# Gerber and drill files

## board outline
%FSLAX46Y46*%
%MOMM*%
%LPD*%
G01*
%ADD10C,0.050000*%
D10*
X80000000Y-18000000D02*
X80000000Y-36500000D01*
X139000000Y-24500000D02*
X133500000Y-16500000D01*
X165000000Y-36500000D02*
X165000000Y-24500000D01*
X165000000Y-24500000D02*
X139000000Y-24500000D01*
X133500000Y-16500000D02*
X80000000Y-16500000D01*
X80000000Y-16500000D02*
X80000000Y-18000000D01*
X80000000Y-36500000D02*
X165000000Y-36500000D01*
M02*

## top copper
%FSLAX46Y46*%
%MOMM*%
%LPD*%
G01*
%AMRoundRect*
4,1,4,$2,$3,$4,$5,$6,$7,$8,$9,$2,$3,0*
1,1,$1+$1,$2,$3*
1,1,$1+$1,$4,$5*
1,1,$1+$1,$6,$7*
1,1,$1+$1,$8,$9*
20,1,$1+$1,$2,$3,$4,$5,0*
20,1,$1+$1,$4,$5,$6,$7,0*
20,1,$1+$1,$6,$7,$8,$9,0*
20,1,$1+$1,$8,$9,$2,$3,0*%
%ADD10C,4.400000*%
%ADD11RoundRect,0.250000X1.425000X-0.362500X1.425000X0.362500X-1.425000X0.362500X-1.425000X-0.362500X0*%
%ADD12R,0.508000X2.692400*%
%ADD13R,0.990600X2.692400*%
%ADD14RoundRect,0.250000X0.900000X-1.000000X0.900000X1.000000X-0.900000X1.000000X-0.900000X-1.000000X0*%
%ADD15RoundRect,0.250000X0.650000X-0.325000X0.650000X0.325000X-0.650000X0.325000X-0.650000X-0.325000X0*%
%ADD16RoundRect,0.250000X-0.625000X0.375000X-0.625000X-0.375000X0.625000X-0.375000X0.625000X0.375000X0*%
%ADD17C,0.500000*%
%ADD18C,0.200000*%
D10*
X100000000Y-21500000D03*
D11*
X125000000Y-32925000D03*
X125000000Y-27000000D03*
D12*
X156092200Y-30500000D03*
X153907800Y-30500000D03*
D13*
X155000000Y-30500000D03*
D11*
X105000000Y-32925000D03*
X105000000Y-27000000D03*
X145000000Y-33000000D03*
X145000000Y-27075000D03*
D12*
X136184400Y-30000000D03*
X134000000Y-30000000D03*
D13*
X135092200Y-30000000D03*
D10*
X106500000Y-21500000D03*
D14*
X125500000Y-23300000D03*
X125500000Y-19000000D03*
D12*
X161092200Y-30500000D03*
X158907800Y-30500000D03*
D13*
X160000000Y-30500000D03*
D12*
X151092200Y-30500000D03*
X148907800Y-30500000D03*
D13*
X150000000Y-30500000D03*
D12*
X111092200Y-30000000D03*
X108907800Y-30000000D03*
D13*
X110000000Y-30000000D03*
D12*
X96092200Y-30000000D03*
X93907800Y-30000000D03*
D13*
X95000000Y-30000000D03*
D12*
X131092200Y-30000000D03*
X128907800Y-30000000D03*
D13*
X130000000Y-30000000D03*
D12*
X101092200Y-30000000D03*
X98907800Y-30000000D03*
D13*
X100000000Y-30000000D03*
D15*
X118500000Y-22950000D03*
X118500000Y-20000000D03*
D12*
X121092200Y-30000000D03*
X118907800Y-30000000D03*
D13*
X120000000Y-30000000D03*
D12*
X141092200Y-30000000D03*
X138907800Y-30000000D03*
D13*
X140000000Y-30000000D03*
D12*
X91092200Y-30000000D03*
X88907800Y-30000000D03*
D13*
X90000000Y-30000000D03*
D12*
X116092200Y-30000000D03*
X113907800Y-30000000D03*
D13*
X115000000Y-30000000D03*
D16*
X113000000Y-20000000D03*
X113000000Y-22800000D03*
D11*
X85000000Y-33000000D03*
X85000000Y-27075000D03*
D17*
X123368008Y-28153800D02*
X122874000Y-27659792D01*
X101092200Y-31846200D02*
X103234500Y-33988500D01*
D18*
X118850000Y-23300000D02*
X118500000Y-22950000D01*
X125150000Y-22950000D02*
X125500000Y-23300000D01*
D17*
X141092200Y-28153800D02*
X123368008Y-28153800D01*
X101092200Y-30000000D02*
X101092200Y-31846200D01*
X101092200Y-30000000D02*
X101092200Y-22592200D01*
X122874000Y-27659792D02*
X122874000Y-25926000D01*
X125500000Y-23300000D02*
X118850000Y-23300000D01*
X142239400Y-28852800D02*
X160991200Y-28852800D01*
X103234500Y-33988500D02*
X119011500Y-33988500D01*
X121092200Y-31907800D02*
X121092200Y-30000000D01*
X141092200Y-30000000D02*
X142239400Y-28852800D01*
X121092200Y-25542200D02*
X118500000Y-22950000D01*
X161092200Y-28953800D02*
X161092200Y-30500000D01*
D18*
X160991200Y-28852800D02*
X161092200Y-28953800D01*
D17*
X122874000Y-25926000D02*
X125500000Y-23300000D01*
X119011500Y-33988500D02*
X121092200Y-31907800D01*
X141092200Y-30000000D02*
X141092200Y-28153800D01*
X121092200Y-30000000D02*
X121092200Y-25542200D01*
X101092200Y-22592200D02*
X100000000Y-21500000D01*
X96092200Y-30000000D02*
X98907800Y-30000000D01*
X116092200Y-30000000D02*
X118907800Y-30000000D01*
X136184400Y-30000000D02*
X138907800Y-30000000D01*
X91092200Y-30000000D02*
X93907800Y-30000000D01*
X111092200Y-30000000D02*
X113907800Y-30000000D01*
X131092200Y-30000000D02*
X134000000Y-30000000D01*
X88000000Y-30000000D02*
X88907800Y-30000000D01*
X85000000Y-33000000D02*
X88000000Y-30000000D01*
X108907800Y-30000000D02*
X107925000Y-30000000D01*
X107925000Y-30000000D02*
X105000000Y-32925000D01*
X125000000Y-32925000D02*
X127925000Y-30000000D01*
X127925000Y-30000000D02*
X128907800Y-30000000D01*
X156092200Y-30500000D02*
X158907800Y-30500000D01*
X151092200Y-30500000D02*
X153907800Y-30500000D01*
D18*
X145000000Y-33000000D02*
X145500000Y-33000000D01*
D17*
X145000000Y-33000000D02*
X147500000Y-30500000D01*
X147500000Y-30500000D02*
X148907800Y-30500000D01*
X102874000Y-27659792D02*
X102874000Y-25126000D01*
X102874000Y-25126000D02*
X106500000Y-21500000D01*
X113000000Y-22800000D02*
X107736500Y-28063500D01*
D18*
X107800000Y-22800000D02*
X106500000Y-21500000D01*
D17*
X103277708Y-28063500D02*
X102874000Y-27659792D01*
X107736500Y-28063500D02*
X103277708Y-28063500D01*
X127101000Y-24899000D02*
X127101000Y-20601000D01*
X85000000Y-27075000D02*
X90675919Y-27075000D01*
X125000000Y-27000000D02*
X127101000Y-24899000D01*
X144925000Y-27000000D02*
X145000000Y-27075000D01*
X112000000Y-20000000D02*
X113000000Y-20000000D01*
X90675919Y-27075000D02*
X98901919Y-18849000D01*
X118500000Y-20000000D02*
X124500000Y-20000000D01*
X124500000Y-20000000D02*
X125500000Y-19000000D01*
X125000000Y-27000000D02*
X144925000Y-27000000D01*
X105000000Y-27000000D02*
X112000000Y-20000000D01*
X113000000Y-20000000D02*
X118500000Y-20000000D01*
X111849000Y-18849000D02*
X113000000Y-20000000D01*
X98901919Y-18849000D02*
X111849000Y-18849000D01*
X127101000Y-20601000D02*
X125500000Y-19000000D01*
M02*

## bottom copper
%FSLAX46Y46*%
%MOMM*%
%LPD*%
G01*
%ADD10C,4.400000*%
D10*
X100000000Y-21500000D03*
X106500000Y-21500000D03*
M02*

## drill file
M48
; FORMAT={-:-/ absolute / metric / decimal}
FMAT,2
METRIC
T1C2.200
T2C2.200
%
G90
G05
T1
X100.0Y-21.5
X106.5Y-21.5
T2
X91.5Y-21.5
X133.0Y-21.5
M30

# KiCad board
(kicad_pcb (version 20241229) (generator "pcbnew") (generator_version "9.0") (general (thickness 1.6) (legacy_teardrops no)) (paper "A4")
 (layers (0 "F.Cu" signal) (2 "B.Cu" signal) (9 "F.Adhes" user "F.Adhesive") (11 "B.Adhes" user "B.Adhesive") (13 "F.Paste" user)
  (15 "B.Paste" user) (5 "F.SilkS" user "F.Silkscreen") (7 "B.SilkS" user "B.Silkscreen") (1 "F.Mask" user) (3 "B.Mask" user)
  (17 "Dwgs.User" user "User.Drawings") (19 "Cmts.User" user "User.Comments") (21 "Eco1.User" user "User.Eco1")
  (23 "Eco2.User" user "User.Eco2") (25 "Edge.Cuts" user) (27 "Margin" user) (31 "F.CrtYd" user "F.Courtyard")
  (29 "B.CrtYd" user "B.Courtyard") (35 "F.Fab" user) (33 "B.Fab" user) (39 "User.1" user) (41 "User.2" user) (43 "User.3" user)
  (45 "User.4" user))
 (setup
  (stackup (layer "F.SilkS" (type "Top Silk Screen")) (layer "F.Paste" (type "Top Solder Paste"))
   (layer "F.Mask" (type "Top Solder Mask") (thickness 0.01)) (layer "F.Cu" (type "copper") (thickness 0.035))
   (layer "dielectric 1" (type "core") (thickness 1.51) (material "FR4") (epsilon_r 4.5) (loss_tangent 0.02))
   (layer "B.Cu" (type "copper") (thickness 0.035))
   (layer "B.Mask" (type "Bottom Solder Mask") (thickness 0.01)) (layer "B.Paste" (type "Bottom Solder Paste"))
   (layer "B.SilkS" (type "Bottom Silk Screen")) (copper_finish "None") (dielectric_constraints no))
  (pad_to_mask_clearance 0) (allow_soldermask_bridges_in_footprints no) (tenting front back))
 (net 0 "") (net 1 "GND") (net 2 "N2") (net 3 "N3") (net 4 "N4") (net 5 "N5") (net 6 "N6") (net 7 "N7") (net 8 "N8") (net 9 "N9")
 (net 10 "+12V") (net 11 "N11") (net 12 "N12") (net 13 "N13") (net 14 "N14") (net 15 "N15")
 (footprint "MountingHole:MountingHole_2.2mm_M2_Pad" (layer "F.Cu") (at 100 21.5)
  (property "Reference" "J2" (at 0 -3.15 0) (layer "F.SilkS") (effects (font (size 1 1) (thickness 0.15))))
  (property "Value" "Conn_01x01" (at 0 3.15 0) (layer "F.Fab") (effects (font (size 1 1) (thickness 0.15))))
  (pad "1" thru_hole circle (at 0 0) (size 4.4 4.4) (drill 2.2) (layers "*.Cu" "*.Mask") (remove_unused_layers no) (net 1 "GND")
   (zone_connect 2)))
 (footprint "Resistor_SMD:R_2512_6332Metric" (layer "F.Cu") (at 125 29.9625 90)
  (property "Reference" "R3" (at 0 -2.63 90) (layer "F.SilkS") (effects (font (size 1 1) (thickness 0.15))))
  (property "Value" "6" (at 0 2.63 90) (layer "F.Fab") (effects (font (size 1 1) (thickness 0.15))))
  (pad "1" smd roundrect (at -2.9625 0 90) (size 1.225 3.35) (layers "F.Cu" "F.Mask" "F.Paste") (roundrect_rratio 0.204082) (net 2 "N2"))
  (pad "2" smd roundrect (at 2.9625 0 90) (size 1.225 3.35) (layers "F.Cu" "F.Mask" "F.Paste") (roundrect_rratio 0.204082) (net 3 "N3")))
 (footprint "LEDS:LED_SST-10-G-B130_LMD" (layer "F.Cu") (at 155 30.5 180)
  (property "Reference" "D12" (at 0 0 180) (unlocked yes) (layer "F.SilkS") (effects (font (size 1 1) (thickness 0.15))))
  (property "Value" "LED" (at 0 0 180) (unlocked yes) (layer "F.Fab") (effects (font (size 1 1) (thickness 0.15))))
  (pad "1" smd rect (at -1.0922 0 180) (size 0.508 2.6924) (layers "F.Cu" "F.Mask" "F.Paste") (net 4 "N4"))
  (pad "2" smd rect (at 1.0922 0 180) (size 0.508 2.6924) (layers "F.Cu" "F.Mask" "F.Paste") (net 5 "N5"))
  (pad "3" smd rect (at 0 0 180) (size 0.9906 2.6924) (layers "F.Cu" "F.Mask" "F.Paste")))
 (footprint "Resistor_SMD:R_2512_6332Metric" (layer "F.Cu") (at 105 29.9625 90)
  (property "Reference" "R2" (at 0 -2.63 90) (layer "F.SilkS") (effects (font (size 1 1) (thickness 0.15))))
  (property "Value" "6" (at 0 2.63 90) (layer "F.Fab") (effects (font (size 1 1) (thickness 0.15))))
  (pad "1" smd roundrect (at -2.9625 0 90) (size 1.225 3.35) (layers "F.Cu" "F.Mask" "F.Paste") (roundrect_rratio 0.204082) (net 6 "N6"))
  (pad "2" smd roundrect (at 2.9625 0 90) (size 1.225 3.35) (layers "F.Cu" "F.Mask" "F.Paste") (roundrect_rratio 0.204082) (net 3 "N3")))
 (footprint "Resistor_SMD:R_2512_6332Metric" (layer "F.Cu") (at 145 30.0375 90)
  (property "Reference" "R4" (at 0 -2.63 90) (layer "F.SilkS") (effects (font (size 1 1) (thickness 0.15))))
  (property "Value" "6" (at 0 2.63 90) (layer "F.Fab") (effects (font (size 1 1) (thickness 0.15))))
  (pad "1" smd roundrect (at -2.9625 0 90) (size 1.225 3.35) (layers "F.Cu" "F.Mask" "F.Paste") (roundrect_rratio 0.204082) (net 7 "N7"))
  (pad "2" smd roundrect (at 2.9625 0 90) (size 1.225 3.35) (layers "F.Cu" "F.Mask" "F.Paste") (roundrect_rratio 0.204082) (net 3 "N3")))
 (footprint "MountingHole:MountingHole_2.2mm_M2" (layer "F.Cu") (at 133 21.5)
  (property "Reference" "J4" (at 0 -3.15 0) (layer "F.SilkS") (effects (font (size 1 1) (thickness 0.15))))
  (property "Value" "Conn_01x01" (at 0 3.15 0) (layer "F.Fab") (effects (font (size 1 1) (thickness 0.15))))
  (pad "" np_thru_hole circle (at 0 0) (size 2.2 2.2) (drill 2.2) (layers "*.Cu" "*.Mask")))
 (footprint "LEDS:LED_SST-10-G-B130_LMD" (layer "F.Cu") (at 135.0922 30 180)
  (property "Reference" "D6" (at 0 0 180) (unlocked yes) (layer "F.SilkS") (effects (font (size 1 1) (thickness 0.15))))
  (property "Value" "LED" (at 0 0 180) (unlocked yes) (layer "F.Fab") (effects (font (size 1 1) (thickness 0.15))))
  (pad "1" smd rect (at -1.0922 0 180) (size 0.508 2.6924) (layers "F.Cu" "F.Mask" "F.Paste") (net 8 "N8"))
  (pad "2" smd rect (at 1.0922 0 180) (size 0.508 2.6924) (layers "F.Cu" "F.Mask" "F.Paste") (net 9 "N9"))
  (pad "3" smd rect (at 0 0 180) (size 0.9906 2.6924) (layers "F.Cu" "F.Mask" "F.Paste")))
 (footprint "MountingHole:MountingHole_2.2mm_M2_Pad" (layer "F.Cu") (at 106.5 21.5)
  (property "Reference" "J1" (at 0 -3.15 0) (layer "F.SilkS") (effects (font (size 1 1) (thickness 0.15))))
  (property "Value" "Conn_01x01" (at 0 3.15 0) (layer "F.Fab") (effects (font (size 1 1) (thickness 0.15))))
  (pad "1" thru_hole circle (at 0 0) (size 4.4 4.4) (drill 2.2) (layers "*.Cu" "*.Mask") (remove_unused_layers no) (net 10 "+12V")
   (zone_connect 2)))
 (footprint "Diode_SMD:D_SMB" (layer "F.Cu") (at 125.5 21.15 90)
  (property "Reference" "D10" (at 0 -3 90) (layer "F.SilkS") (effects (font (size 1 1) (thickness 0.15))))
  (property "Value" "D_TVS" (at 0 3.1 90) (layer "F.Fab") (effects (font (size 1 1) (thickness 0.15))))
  (pad "1" smd roundrect (at -2.15 0 90) (size 2.5 2.3) (layers "F.Cu" "F.Mask" "F.Paste") (roundrect_rratio 0.1086956522) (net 1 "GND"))
  (pad "2" smd roundrect (at 2.15 0 90) (size 2.5 2.3) (layers "F.Cu" "F.Mask" "F.Paste") (roundrect_rratio 0.1086956522) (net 3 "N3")))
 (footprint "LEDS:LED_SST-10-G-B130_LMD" (layer "F.Cu") (at 160 30.5 180)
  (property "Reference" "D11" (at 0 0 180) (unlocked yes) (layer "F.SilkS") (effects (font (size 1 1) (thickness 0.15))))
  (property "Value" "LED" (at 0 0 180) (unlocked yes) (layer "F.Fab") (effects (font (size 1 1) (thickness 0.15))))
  (pad "1" smd rect (at -1.0922 0 180) (size 0.508 2.6924) (layers "F.Cu" "F.Mask" "F.Paste") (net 1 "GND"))
  (pad "2" smd rect (at 1.0922 0 180) (size 0.508 2.6924) (layers "F.Cu" "F.Mask" "F.Paste") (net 4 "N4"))
  (pad "3" smd rect (at 0 0 180) (size 0.9906 2.6924) (layers "F.Cu" "F.Mask" "F.Paste")))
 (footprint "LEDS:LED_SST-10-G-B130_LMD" (layer "F.Cu") (at 150 30.5 180)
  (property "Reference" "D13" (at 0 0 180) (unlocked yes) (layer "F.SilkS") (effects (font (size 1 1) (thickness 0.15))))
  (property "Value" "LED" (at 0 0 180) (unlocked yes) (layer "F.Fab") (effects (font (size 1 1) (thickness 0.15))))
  (pad "1" smd rect (at -1.0922 0 180) (size 0.508 2.6924) (layers "F.Cu" "F.Mask" "F.Paste") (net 5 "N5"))
  (pad "2" smd rect (at 1.0922 0 180) (size 0.508 2.6924) (layers "F.Cu" "F.Mask" "F.Paste") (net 7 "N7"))
  (pad "3" smd rect (at 0 0 180) (size 0.9906 2.6924) (layers "F.Cu" "F.Mask" "F.Paste")))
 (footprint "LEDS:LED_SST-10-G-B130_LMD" (layer "F.Cu") (at 110 30 180)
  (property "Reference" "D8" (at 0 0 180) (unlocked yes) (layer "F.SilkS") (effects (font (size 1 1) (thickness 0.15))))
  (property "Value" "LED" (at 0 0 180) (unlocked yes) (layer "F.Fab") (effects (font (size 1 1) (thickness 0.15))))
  (pad "1" smd rect (at -1.0922 0 180) (size 0.508 2.6924) (layers "F.Cu" "F.Mask" "F.Paste") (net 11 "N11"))
  (pad "2" smd rect (at 1.0922 0 180) (size 0.508 2.6924) (layers "F.Cu" "F.Mask" "F.Paste") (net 6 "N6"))
  (pad "3" smd rect (at 0 0 180) (size 0.9906 2.6924) (layers "F.Cu" "F.Mask" "F.Paste")))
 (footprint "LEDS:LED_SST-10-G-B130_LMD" (layer "F.Cu") (at 95 30 180)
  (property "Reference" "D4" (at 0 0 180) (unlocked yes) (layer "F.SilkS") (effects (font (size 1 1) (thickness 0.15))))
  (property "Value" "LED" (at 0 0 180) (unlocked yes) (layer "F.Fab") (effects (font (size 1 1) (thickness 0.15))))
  (pad "1" smd rect (at -1.0922 0 180) (size 0.508 2.6924) (layers "F.Cu" "F.Mask" "F.Paste") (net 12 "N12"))
  (pad "2" smd rect (at 1.0922 0 180) (size 0.508 2.6924) (layers "F.Cu" "F.Mask" "F.Paste") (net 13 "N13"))
  (pad "3" smd rect (at 0 0 180) (size 0.9906 2.6924) (layers "F.Cu" "F.Mask" "F.Paste")))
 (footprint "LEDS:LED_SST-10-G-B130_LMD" (layer "F.Cu") (at 130 30 180)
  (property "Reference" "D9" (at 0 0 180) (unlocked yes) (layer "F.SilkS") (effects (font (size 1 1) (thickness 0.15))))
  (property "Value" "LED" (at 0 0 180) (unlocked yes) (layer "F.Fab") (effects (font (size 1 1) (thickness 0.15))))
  (pad "1" smd rect (at -1.0922 0 180) (size 0.508 2.6924) (layers "F.Cu" "F.Mask" "F.Paste") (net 9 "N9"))
  (pad "2" smd rect (at 1.0922 0 180) (size 0.508 2.6924) (layers "F.Cu" "F.Mask" "F.Paste") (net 2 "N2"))
  (pad "3" smd rect (at 0 0 180) (size 0.9906 2.6924) (layers "F.Cu" "F.Mask" "F.Paste")))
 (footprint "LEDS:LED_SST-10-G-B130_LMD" (layer "F.Cu") (at 100 30 180)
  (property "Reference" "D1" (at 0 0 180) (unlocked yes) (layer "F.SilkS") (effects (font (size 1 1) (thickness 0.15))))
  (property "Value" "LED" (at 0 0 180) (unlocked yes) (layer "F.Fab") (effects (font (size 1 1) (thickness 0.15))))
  (pad "1" smd rect (at -1.0922 0 180) (size 0.508 2.6924) (layers "F.Cu" "F.Mask" "F.Paste") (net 1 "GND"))
  (pad "2" smd rect (at 1.0922 0 180) (size 0.508 2.6924) (layers "F.Cu" "F.Mask" "F.Paste") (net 12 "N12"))
  (pad "3" smd rect (at 0 0 180) (size 0.9906 2.6924) (layers "F.Cu" "F.Mask" "F.Paste")))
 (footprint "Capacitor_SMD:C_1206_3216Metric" (layer "F.Cu") (at 118.5 21.475 90)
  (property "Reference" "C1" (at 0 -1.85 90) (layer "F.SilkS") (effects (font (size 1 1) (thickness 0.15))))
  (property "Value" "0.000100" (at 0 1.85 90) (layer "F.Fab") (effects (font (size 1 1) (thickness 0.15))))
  (pad "1" smd roundrect (at -1.475 0 90) (size 1.15 1.8) (layers "F.Cu" "F.Mask" "F.Paste") (roundrect_rratio 0.217391) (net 1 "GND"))
  (pad "2" smd roundrect (at 1.475 0 90) (size 1.15 1.8) (layers "F.Cu" "F.Mask" "F.Paste") (roundrect_rratio 0.217391) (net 3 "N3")))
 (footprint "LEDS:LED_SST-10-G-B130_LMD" (layer "F.Cu") (at 120 30 180)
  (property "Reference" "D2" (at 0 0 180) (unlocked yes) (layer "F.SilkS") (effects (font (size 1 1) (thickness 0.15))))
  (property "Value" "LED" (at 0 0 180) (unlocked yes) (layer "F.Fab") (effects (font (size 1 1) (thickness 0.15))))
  (pad "1" smd rect (at -1.0922 0 180) (size 0.508 2.6924) (layers "F.Cu" "F.Mask" "F.Paste") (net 1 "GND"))
  (pad "2" smd rect (at 1.0922 0 180) (size 0.508 2.6924) (layers "F.Cu" "F.Mask" "F.Paste") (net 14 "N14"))
  (pad "3" smd rect (at 0 0 180) (size 0.9906 2.6924) (layers "F.Cu" "F.Mask" "F.Paste")))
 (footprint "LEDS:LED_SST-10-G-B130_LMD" (layer "F.Cu") (at 140 30 180)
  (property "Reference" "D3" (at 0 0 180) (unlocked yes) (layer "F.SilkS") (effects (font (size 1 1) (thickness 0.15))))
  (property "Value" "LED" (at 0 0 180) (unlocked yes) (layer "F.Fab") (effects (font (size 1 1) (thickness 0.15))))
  (pad "1" smd rect (at -1.0922 0 180) (size 0.508 2.6924) (layers "F.Cu" "F.Mask" "F.Paste") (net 1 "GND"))
  (pad "2" smd rect (at 1.0922 0 180) (size 0.508 2.6924) (layers "F.Cu" "F.Mask" "F.Paste") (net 8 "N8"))
  (pad "3" smd rect (at 0 0 180) (size 0.9906 2.6924) (layers "F.Cu" "F.Mask" "F.Paste")))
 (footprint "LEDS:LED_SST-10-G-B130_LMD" (layer "F.Cu") (at 90 30 180)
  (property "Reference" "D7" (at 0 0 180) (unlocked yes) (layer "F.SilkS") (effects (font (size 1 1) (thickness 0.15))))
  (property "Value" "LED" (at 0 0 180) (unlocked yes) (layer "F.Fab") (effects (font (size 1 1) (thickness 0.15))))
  (pad "1" smd rect (at -1.0922 0 180) (size 0.508 2.6924) (layers "F.Cu" "F.Mask" "F.Paste") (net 13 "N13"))
  (pad "2" smd rect (at 1.0922 0 180) (size 0.508 2.6924) (layers "F.Cu" "F.Mask" "F.Paste") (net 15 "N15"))
  (pad "3" smd rect (at 0 0 180) (size 0.9906 2.6924) (layers "F.Cu" "F.Mask" "F.Paste")))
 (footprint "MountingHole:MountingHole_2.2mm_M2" (layer "F.Cu") (at 91.5 21.5)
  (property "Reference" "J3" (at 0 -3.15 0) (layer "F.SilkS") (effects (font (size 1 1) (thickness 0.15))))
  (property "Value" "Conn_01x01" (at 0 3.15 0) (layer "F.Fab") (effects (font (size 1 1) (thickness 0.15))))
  (pad "" np_thru_hole circle (at 0 0) (size 2.2 2.2) (drill 2.2) (layers "*.Cu" "*.Mask")))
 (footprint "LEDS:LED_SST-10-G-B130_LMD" (layer "F.Cu") (at 115 30 180)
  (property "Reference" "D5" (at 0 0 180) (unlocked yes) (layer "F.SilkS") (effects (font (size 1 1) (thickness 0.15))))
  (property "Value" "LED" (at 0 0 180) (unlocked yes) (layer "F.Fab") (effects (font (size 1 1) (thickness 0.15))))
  (pad "1" smd rect (at -1.0922 0 180) (size 0.508 2.6924) (layers "F.Cu" "F.Mask" "F.Paste") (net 14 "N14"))
  (pad "2" smd rect (at 1.0922 0 180) (size 0.508 2.6924) (layers "F.Cu" "F.Mask" "F.Paste") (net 11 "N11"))
  (pad "3" smd rect (at 0 0 180) (size 0.9906 2.6924) (layers "F.Cu" "F.Mask" "F.Paste")))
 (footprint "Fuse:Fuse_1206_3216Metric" (layer "F.Cu") (at 113 21.4 -90)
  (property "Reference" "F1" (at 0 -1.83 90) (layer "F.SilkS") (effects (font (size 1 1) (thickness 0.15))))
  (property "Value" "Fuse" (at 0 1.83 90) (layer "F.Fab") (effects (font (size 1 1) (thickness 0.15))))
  (pad "1" smd roundrect (at -1.4 0 270) (size 1.25 1.75) (layers "F.Cu" "F.Mask" "F.Paste") (roundrect_rratio 0.2) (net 3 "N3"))
  (pad "2" smd roundrect (at 1.4 0 270) (size 1.25 1.75) (layers "F.Cu" "F.Mask" "F.Paste") (roundrect_rratio 0.2) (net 10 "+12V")))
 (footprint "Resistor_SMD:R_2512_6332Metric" (layer "F.Cu") (at 85 30.0375 90)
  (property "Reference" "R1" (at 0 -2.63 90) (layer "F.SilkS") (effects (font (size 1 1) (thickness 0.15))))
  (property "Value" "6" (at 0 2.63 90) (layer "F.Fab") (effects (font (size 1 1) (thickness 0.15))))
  (pad "1" smd roundrect (at -2.9625 0 90) (size 1.225 3.35) (layers "F.Cu" "F.Mask" "F.Paste") (roundrect_rratio 0.204082) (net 15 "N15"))
  (pad "2" smd roundrect (at 2.9625 0 90) (size 1.225 3.35) (layers "F.Cu" "F.Mask" "F.Paste") (roundrect_rratio 0.204082) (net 3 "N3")))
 (gr_line (start 80 18) (end 80 36.5) (stroke (width 0.05) (type default)) (layer "Edge.Cuts"))
 (gr_line (start 139 24.5) (end 133.5 16.5) (stroke (width 0.05) (type default)) (layer "Edge.Cuts"))
 (gr_line (start 165 36.5) (end 165 24.5) (stroke (width 0.05) (type default)) (layer "Edge.Cuts"))
 (gr_line (start 165 24.5) (end 139 24.5) (stroke (width 0.05) (type default)) (layer "Edge.Cuts"))
 (gr_line (start 133.5 16.5) (end 80 16.5) (stroke (width 0.05) (type default)) (layer "Edge.Cuts"))
 (gr_line (start 80 16.5) (end 80 18) (stroke (width 0.05) (type default)) (layer "Edge.Cuts"))
 (gr_line (start 80 36.5) (end 165 36.5) (stroke (width 0.05) (type default)) (layer "Edge.Cuts"))
 (segment (start 123.368008 28.1538) (end 122.874 27.659792) (width 0.5) (layer "F.Cu") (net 1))
 (segment (start 101.0922 31.8462) (end 103.2345 33.9885) (width 0.5) (layer "F.Cu") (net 1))
 (segment (start 118.85 23.3) (end 118.5 22.95) (width 0.2) (layer "F.Cu") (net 1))
 (segment (start 125.15 22.95) (end 125.5 23.3) (width 0.2) (layer "F.Cu") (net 1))
 (segment (start 141.0922 28.1538) (end 123.368008 28.1538) (width 0.5) (layer "F.Cu") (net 1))
 (segment (start 101.0922 30) (end 101.0922 31.8462) (width 0.5) (layer "F.Cu") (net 1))
 (segment (start 101.0922 30) (end 101.0922 22.5922) (width 0.5) (layer "F.Cu") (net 1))
 (segment (start 122.874 27.659792) (end 122.874 25.926) (width 0.5) (layer "F.Cu") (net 1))
 (segment (start 125.5 23.3) (end 118.85 23.3) (width 0.5) (layer "F.Cu") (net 1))
 (segment (start 142.2394 28.8528) (end 160.9912 28.8528) (width 0.5) (layer "F.Cu") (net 1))
 (segment (start 103.2345 33.9885) (end 119.0115 33.9885) (width 0.5) (layer "F.Cu") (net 1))
 (segment (start 121.0922 31.9078) (end 121.0922 30) (width 0.5) (layer "F.Cu") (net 1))
 (segment (start 141.0922 30) (end 142.2394 28.8528) (width 0.5) (layer "F.Cu") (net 1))
 (segment (start 121.0922 25.5422) (end 118.5 22.95) (width 0.5) (layer "F.Cu") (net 1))
 (segment (start 161.0922 28.9538) (end 161.0922 30.5) (width 0.5) (layer "F.Cu") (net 1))
 (segment (start 160.9912 28.8528) (end 161.0922 28.9538) (width 0.2) (layer "F.Cu") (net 1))
 (segment (start 122.874 25.926) (end 125.5 23.3) (width 0.5) (layer "F.Cu") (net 1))
 (segment (start 119.0115 33.9885) (end 121.0922 31.9078) (width 0.5) (layer "F.Cu") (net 1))
 (segment (start 141.0922 30) (end 141.0922 28.1538) (width 0.5) (layer "F.Cu") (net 1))
 (segment (start 121.0922 30) (end 121.0922 25.5422) (width 0.5) (layer "F.Cu") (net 1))
 (segment (start 101.0922 22.5922) (end 100 21.5) (width 0.5) (layer "F.Cu") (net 1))
 (segment (start 96.0922 30) (end 98.9078 30) (width 0.5) (layer "F.Cu") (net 12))
 (segment (start 116.0922 30) (end 118.9078 30) (width 0.5) (layer "F.Cu") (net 14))
 (segment (start 136.1844 30) (end 138.9078 30) (width 0.5) (layer "F.Cu") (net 8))
 (segment (start 91.0922 30) (end 93.9078 30) (width 0.5) (layer "F.Cu") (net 13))
 (segment (start 111.0922 30) (end 113.9078 30) (width 0.5) (layer "F.Cu") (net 11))
 (segment (start 131.0922 30) (end 134 30) (width 0.5) (layer "F.Cu") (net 9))
 (segment (start 88 30) (end 88.9078 30) (width 0.5) (layer "F.Cu") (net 15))
 (segment (start 85 33) (end 88 30) (width 0.5) (layer "F.Cu") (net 15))
 (segment (start 108.9078 30) (end 107.925 30) (width 0.5) (layer "F.Cu") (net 6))
 (segment (start 107.925 30) (end 105 32.925) (width 0.5) (layer "F.Cu") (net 6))
 (segment (start 125 32.925) (end 127.925 30) (width 0.5) (layer "F.Cu") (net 2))
 (segment (start 127.925 30) (end 128.9078 30) (width 0.5) (layer "F.Cu") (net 2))
 (segment (start 156.0922 30.5) (end 158.9078 30.5) (width 0.5) (layer "F.Cu") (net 4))
 (segment (start 151.0922 30.5) (end 153.9078 30.5) (width 0.5) (layer "F.Cu") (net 5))
 (segment (start 145 33) (end 145.5 33) (width 0.2) (layer "F.Cu") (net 7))
 (segment (start 145 33) (end 147.5 30.5) (width 0.5) (layer "F.Cu") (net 7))
 (segment (start 147.5 30.5) (end 148.9078 30.5) (width 0.5) (layer "F.Cu") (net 7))
 (segment (start 102.874 27.659792) (end 102.874 25.126) (width 0.5) (layer "F.Cu") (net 10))
 (segment (start 102.874 25.126) (end 106.5 21.5) (width 0.5) (layer "F.Cu") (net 10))
 (segment (start 113 22.8) (end 107.7365 28.0635) (width 0.5) (layer "F.Cu") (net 10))
 (segment (start 107.8 22.8) (end 106.5 21.5) (width 0.2) (layer "F.Cu") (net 10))
 (segment (start 103.277708 28.0635) (end 102.874 27.659792) (width 0.5) (layer "F.Cu") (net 10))
 (segment (start 107.7365 28.0635) (end 103.277708 28.0635) (width 0.5) (layer "F.Cu") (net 10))
 (segment (start 127.101 24.899) (end 127.101 20.601) (width 0.5) (layer "F.Cu") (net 3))
 (segment (start 85 27.075) (end 90.675919 27.075) (width 0.5) (layer "F.Cu") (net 3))
 (segment (start 125 27) (end 127.101 24.899) (width 0.5) (layer "F.Cu") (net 3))
 (segment (start 144.925 27) (end 145 27.075) (width 0.5) (layer "F.Cu") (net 3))
 (segment (start 112 20) (end 113 20) (width 0.5) (layer "F.Cu") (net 3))
 (segment (start 90.675919 27.075) (end 98.901919 18.849) (width 0.5) (layer "F.Cu") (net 3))
 (segment (start 118.5 20) (end 124.5 20) (width 0.5) (layer "F.Cu") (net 3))
 (segment (start 124.5 20) (end 125.5 19) (width 0.5) (layer "F.Cu") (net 3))
 (segment (start 125 27) (end 144.925 27) (width 0.5) (layer "F.Cu") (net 3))
 (segment (start 105 27) (end 112 20) (width 0.5) (layer "F.Cu") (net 3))
 (segment (start 113 20) (end 118.5 20) (width 0.5) (layer "F.Cu") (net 3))
 (segment (start 111.849 18.849) (end 113 20) (width 0.5) (layer "F.Cu") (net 3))
 (segment (start 98.901919 18.849) (end 111.849 18.849) (width 0.5) (layer "F.Cu") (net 3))
 (segment (start 127.101 20.601) (end 125.5 19) (width 0.5) (layer "F.Cu") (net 3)))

